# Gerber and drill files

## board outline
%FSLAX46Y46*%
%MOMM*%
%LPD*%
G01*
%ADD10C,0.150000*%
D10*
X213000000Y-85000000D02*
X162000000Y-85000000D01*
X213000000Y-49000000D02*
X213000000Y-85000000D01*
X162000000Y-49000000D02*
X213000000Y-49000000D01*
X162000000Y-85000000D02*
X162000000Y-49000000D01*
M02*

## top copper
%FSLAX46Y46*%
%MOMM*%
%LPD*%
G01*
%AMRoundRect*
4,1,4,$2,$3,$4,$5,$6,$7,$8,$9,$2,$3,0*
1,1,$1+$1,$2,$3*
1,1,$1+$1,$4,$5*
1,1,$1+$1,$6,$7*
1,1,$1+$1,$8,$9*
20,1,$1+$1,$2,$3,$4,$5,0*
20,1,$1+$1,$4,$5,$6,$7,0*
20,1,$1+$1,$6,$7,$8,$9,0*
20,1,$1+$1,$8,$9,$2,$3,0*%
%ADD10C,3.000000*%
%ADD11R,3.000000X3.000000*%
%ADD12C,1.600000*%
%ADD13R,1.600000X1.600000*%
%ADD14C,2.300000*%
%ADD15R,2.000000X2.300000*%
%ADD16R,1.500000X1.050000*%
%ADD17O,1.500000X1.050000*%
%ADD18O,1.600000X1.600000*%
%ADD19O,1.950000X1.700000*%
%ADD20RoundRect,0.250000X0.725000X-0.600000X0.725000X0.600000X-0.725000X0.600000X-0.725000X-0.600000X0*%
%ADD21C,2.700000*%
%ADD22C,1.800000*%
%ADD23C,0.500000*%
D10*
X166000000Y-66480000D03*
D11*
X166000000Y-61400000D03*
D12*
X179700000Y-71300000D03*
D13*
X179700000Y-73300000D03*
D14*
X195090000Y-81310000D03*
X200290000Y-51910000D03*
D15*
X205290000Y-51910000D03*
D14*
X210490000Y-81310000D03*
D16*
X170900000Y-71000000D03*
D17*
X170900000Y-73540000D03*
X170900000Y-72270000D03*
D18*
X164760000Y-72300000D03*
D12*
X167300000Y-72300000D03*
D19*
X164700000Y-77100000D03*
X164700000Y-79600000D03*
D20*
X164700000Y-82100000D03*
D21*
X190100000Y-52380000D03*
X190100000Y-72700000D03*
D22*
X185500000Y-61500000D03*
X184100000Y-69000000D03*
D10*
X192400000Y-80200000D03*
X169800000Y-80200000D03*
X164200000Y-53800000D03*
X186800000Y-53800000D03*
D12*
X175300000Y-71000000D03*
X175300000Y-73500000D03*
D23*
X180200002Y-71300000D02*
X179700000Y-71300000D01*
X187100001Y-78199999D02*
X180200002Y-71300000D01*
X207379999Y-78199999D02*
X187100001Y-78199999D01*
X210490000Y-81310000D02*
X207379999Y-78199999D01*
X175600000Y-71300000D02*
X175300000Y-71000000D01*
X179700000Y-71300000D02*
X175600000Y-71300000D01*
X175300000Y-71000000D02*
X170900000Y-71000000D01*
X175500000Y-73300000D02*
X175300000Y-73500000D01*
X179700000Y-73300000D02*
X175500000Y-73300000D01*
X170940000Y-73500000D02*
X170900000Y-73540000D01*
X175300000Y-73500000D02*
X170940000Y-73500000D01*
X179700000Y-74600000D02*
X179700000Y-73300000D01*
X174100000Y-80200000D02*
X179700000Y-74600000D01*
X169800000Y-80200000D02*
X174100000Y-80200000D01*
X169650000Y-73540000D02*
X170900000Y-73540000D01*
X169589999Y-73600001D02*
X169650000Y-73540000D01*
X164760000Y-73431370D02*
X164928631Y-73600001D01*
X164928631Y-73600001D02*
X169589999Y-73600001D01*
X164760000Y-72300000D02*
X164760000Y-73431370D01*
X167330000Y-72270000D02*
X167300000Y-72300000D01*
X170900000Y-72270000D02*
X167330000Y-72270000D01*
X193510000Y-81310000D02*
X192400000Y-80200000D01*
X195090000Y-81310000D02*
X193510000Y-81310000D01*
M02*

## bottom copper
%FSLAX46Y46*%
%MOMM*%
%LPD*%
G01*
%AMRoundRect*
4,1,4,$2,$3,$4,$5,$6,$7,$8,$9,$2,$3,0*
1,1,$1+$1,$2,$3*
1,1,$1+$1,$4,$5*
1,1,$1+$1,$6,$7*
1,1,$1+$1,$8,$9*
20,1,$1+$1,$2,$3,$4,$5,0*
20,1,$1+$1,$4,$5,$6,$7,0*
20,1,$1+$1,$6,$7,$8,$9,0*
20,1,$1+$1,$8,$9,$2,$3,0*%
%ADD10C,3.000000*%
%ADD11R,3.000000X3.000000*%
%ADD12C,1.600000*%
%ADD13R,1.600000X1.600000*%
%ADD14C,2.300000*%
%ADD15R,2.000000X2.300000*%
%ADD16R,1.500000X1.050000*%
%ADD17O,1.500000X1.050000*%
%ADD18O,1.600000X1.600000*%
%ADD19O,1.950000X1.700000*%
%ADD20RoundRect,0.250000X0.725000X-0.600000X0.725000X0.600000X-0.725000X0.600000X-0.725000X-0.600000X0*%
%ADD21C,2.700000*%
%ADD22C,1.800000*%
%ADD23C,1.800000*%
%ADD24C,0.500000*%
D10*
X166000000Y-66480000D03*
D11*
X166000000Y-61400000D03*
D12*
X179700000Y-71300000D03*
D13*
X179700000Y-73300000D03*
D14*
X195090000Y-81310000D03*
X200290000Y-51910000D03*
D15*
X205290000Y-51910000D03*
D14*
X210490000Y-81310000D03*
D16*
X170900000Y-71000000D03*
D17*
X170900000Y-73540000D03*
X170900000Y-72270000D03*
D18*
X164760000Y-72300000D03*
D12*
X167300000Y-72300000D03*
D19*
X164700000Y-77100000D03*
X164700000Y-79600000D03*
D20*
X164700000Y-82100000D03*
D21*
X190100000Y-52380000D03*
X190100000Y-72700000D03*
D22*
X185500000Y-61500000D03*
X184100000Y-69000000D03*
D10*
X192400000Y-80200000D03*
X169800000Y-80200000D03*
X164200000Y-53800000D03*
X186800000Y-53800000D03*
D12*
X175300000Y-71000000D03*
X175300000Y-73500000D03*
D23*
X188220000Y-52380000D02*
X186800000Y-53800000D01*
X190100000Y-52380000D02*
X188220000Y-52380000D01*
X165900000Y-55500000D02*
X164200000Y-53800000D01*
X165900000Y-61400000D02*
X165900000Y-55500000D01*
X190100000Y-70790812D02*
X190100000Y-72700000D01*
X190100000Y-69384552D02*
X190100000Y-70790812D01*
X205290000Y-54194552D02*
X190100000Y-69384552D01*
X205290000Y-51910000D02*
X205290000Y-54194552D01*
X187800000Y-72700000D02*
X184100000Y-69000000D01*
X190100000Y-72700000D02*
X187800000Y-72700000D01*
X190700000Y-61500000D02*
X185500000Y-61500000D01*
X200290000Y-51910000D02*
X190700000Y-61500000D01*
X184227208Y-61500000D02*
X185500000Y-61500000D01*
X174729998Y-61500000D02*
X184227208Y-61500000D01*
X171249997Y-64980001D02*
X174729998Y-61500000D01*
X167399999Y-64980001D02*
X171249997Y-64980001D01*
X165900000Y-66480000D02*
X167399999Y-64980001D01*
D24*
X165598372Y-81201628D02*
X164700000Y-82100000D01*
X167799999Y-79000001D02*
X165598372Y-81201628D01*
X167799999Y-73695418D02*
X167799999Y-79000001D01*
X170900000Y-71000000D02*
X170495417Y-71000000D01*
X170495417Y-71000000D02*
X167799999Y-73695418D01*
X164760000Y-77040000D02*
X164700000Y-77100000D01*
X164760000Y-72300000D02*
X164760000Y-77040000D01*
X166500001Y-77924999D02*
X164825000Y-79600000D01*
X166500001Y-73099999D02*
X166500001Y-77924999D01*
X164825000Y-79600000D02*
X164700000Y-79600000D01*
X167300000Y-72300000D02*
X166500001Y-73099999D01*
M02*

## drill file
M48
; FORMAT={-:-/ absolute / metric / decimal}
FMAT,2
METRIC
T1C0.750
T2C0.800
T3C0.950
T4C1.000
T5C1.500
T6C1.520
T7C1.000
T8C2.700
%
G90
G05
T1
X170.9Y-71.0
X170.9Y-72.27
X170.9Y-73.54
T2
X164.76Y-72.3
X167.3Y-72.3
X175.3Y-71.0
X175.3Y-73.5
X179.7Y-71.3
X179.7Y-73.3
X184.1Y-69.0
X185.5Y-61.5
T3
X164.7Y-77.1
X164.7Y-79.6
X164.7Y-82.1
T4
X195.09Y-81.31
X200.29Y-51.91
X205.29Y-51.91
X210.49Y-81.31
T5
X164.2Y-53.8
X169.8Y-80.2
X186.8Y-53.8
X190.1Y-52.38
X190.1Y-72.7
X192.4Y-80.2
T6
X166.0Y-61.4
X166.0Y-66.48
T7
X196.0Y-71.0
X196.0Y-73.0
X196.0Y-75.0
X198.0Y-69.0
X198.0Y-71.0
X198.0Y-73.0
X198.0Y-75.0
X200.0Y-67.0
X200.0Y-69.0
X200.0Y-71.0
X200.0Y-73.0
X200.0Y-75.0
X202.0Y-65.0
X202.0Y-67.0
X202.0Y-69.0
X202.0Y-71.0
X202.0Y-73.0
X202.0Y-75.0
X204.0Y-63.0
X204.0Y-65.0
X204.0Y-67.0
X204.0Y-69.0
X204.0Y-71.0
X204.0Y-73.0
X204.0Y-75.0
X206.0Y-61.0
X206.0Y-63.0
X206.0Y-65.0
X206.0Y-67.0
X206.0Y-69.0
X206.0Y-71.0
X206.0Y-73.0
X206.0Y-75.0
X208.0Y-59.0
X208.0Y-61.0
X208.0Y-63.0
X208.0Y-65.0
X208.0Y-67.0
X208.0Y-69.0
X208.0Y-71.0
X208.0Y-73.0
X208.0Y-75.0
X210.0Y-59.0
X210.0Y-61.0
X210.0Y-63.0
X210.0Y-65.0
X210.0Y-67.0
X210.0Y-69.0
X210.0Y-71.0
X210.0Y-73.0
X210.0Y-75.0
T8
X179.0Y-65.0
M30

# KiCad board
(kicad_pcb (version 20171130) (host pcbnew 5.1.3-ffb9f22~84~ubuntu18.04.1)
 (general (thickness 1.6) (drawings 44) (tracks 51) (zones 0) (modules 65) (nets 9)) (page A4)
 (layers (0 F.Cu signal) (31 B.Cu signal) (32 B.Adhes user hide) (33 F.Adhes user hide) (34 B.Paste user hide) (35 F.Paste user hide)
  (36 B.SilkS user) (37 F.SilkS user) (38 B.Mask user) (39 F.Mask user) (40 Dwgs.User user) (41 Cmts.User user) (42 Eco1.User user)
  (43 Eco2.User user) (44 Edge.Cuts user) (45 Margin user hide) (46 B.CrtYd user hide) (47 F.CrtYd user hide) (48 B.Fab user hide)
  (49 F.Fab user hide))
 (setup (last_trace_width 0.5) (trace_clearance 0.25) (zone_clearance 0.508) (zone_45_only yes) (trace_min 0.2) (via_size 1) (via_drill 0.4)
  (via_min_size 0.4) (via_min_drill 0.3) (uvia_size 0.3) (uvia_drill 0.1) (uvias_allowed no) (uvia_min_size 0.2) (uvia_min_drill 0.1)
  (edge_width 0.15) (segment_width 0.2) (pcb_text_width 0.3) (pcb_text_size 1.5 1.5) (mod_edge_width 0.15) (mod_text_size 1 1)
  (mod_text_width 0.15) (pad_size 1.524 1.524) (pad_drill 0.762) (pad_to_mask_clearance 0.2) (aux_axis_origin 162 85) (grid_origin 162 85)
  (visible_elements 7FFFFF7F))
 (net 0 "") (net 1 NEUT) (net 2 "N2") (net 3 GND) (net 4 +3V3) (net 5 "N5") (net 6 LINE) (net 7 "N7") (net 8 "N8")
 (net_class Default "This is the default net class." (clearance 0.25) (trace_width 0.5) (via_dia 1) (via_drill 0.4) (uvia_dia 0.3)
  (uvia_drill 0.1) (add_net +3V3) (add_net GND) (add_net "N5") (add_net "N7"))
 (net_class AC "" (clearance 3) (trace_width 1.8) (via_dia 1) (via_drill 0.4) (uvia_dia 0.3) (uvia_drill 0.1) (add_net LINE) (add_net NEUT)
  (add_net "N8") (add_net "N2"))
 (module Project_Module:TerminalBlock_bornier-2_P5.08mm (layer F.Cu) (at 166 61.4 270)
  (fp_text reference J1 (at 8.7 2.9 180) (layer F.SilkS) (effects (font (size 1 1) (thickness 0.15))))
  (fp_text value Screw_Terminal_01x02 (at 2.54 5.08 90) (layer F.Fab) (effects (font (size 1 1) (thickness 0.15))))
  (pad 2 thru_hole circle (at 5.08 0 270) (size 3 3) (drill 1.52) (layers *.Cu *.Mask) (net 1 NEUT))
  (pad 1 thru_hole rect (at 0 0 270) (size 3 3) (drill 1.52) (layers *.Cu *.Mask) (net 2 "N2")))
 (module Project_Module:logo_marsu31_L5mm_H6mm (layer B.Cu) (at 173.8 80.9 180)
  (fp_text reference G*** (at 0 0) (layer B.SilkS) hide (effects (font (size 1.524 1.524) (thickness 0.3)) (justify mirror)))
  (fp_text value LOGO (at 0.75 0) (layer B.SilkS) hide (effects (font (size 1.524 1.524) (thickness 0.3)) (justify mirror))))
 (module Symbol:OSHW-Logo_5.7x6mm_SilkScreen (layer B.Cu) (at 202.9 80.9 180)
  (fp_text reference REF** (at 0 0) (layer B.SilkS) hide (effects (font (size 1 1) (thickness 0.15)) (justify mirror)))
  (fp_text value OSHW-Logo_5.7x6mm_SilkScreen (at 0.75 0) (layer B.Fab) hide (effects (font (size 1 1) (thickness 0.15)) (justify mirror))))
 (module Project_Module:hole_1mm (layer F.Cu) (at 210 75)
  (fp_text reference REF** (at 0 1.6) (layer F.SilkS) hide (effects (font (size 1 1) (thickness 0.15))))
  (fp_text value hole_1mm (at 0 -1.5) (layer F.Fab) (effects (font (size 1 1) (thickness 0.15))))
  (pad "" np_thru_hole circle (at 0 0) (size 1 1) (drill 1) (layers *.Cu *.Mask)))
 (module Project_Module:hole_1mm (layer F.Cu) (at 208 75)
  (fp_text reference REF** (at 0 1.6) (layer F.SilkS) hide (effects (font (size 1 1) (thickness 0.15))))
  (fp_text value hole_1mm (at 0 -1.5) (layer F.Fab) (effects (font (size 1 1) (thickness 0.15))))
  (pad "" np_thru_hole circle (at 0 0) (size 1 1) (drill 1) (layers *.Cu *.Mask)))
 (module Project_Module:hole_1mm (layer F.Cu) (at 206 75)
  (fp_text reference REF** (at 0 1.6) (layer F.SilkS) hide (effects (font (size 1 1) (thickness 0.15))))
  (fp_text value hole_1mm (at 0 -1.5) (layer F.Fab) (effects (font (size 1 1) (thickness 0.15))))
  (pad "" np_thru_hole circle (at 0 0) (size 1 1) (drill 1) (layers *.Cu *.Mask)))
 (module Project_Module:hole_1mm (layer F.Cu) (at 204 75)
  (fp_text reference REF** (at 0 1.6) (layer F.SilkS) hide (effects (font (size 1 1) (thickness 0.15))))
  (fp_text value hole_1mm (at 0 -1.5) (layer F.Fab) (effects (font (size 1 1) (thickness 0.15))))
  (pad "" np_thru_hole circle (at 0 0) (size 1 1) (drill 1) (layers *.Cu *.Mask)))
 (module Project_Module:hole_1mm (layer F.Cu) (at 202 75)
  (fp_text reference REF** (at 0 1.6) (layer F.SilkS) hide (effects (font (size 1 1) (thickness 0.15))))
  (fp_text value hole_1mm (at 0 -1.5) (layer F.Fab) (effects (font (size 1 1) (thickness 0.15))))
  (pad "" np_thru_hole circle (at 0 0) (size 1 1) (drill 1) (layers *.Cu *.Mask)))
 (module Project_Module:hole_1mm (layer F.Cu) (at 200 75)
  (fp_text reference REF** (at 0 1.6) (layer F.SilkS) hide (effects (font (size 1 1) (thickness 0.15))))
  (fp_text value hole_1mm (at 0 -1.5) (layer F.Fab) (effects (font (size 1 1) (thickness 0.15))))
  (pad "" np_thru_hole circle (at 0 0) (size 1 1) (drill 1) (layers *.Cu *.Mask)))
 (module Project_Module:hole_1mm (layer F.Cu) (at 198 75)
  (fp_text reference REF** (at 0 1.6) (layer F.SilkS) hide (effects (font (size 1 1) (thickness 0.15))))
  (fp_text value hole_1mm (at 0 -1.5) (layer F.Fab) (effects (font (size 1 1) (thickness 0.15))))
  (pad "" np_thru_hole circle (at 0 0) (size 1 1) (drill 1) (layers *.Cu *.Mask)))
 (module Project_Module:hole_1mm (layer F.Cu) (at 196 75)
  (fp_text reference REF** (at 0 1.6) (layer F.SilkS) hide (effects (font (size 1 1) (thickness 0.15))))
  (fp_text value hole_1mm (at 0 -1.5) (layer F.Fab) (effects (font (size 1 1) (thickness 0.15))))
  (pad "" np_thru_hole circle (at 0 0) (size 1 1) (drill 1) (layers *.Cu *.Mask)))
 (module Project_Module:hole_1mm (layer F.Cu) (at 210 73)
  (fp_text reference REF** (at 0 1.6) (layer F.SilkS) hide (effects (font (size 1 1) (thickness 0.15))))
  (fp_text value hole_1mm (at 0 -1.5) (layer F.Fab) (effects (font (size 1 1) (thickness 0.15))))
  (pad "" np_thru_hole circle (at 0 0) (size 1 1) (drill 1) (layers *.Cu *.Mask)))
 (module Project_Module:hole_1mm (layer F.Cu) (at 208 73)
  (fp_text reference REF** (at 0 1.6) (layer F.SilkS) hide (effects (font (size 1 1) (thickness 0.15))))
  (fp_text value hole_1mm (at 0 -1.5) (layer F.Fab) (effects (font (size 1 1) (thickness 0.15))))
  (pad "" np_thru_hole circle (at 0 0) (size 1 1) (drill 1) (layers *.Cu *.Mask)))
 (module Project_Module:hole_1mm (layer F.Cu) (at 206 73)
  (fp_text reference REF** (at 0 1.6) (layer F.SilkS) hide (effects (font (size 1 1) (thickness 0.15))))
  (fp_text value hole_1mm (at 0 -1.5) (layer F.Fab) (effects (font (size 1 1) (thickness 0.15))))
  (pad "" np_thru_hole circle (at 0 0) (size 1 1) (drill 1) (layers *.Cu *.Mask)))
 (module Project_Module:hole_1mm (layer F.Cu) (at 204 73)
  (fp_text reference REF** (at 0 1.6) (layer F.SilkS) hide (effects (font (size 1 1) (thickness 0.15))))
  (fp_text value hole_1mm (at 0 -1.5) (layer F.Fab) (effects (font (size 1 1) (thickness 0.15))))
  (pad "" np_thru_hole circle (at 0 0) (size 1 1) (drill 1) (layers *.Cu *.Mask)))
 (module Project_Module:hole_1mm (layer F.Cu) (at 202 73)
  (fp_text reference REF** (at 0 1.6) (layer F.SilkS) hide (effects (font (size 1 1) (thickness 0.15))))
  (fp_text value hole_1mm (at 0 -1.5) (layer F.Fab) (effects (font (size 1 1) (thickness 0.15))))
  (pad "" np_thru_hole circle (at 0 0) (size 1 1) (drill 1) (layers *.Cu *.Mask)))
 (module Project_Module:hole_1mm (layer F.Cu) (at 200 73)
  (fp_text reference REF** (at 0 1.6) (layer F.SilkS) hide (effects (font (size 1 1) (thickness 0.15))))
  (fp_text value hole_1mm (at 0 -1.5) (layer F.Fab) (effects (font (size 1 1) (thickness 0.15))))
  (pad "" np_thru_hole circle (at 0 0) (size 1 1) (drill 1) (layers *.Cu *.Mask)))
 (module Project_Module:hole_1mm (layer F.Cu) (at 198 73)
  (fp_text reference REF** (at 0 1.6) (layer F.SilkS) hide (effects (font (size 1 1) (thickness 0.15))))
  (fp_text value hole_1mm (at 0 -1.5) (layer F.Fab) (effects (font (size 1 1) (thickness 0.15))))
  (pad "" np_thru_hole circle (at 0 0) (size 1 1) (drill 1) (layers *.Cu *.Mask)))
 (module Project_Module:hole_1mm (layer F.Cu) (at 196 73)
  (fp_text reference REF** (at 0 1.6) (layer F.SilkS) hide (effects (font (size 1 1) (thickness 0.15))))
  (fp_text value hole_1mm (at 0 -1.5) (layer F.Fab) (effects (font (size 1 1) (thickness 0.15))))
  (pad "" np_thru_hole circle (at 0 0) (size 1 1) (drill 1) (layers *.Cu *.Mask)))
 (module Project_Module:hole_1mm (layer F.Cu) (at 210 71)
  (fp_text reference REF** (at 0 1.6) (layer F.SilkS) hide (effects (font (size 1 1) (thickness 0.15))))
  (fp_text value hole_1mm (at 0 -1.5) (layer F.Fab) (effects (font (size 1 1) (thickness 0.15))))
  (pad "" np_thru_hole circle (at 0 0) (size 1 1) (drill 1) (layers *.Cu *.Mask)))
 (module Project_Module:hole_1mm (layer F.Cu) (at 208 71)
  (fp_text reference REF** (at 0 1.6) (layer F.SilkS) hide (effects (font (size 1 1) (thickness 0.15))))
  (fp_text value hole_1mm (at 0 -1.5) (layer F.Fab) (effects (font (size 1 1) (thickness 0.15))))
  (pad "" np_thru_hole circle (at 0 0) (size 1 1) (drill 1) (layers *.Cu *.Mask)))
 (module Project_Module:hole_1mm (layer F.Cu) (at 206 71)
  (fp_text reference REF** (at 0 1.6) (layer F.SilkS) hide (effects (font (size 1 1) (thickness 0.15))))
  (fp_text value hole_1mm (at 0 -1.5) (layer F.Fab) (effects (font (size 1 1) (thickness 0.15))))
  (pad "" np_thru_hole circle (at 0 0) (size 1 1) (drill 1) (layers *.Cu *.Mask)))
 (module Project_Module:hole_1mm (layer F.Cu) (at 204 71)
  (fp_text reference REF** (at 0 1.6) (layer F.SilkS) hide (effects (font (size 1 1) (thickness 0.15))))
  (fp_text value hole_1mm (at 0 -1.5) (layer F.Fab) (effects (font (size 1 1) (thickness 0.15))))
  (pad "" np_thru_hole circle (at 0 0) (size 1 1) (drill 1) (layers *.Cu *.Mask)))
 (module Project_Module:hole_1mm (layer F.Cu) (at 202 71)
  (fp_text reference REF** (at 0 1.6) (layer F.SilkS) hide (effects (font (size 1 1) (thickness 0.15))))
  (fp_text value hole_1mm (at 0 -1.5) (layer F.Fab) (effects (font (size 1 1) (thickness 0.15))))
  (pad "" np_thru_hole circle (at 0 0) (size 1 1) (drill 1) (layers *.Cu *.Mask)))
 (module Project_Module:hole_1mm (layer F.Cu) (at 200 71)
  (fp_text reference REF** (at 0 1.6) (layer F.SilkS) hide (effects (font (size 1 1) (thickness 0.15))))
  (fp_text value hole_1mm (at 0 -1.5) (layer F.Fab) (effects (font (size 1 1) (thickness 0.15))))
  (pad "" np_thru_hole circle (at 0 0) (size 1 1) (drill 1) (layers *.Cu *.Mask)))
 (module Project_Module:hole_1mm (layer F.Cu) (at 198 71)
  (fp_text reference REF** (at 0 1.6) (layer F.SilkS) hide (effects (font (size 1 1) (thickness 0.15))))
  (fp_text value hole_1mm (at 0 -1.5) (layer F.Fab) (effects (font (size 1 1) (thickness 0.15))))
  (pad "" np_thru_hole circle (at 0 0) (size 1 1) (drill 1) (layers *.Cu *.Mask)))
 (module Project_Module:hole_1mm (layer F.Cu) (at 196 71)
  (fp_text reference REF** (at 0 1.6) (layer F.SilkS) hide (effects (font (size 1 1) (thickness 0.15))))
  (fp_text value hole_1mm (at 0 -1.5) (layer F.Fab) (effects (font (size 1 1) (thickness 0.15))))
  (pad "" np_thru_hole circle (at 0 0) (size 1 1) (drill 1) (layers *.Cu *.Mask)))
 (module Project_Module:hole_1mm (layer F.Cu) (at 210 69)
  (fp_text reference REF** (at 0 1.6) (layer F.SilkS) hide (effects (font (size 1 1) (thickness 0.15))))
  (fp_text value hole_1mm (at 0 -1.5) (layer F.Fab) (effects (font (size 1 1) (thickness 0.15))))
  (pad "" np_thru_hole circle (at 0 0) (size 1 1) (drill 1) (layers *.Cu *.Mask)))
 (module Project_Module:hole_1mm (layer F.Cu) (at 208 69)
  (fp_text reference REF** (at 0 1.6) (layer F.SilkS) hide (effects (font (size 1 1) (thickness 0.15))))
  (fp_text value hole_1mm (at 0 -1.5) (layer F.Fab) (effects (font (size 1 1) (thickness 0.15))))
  (pad "" np_thru_hole circle (at 0 0) (size 1 1) (drill 1) (layers *.Cu *.Mask)))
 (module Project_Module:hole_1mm (layer F.Cu) (at 206 69)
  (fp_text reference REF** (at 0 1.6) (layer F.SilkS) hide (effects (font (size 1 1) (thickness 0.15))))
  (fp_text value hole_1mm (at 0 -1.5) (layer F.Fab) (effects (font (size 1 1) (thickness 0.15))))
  (pad "" np_thru_hole circle (at 0 0) (size 1 1) (drill 1) (layers *.Cu *.Mask)))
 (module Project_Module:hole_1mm (layer F.Cu) (at 204 69)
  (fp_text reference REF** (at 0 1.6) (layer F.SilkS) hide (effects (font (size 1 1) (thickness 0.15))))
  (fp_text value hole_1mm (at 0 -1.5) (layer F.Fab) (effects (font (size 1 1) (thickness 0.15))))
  (pad "" np_thru_hole circle (at 0 0) (size 1 1) (drill 1) (layers *.Cu *.Mask)))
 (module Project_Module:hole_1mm (layer F.Cu) (at 202 69)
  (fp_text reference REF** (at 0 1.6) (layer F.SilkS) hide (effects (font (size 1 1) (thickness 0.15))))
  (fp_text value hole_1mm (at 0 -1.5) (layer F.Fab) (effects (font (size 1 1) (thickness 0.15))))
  (pad "" np_thru_hole circle (at 0 0) (size 1 1) (drill 1) (layers *.Cu *.Mask)))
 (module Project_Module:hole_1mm (layer F.Cu) (at 200 69)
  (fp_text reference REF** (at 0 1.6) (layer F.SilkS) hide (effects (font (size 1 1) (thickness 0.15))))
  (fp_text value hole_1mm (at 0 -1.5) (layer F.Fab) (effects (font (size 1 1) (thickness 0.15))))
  (pad "" np_thru_hole circle (at 0 0) (size 1 1) (drill 1) (layers *.Cu *.Mask)))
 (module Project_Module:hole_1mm (layer F.Cu) (at 198 69)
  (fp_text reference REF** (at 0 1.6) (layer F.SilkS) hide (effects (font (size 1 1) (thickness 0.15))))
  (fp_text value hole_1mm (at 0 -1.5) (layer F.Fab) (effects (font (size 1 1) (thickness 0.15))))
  (pad "" np_thru_hole circle (at 0 0) (size 1 1) (drill 1) (layers *.Cu *.Mask)))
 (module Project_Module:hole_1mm (layer F.Cu) (at 210 67)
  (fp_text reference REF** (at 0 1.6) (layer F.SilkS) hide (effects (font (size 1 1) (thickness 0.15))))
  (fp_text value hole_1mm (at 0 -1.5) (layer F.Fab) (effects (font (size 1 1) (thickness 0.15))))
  (pad "" np_thru_hole circle (at 0 0) (size 1 1) (drill 1) (layers *.Cu *.Mask)))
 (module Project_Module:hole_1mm (layer F.Cu) (at 208 67)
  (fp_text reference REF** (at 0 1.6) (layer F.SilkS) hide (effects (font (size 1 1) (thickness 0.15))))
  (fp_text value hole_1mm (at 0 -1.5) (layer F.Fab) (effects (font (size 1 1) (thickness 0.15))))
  (pad "" np_thru_hole circle (at 0 0) (size 1 1) (drill 1) (layers *.Cu *.Mask)))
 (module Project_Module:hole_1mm (layer F.Cu) (at 206 67)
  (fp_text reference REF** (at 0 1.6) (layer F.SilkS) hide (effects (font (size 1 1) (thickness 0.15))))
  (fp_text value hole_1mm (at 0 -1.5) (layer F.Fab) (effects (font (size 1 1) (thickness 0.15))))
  (pad "" np_thru_hole circle (at 0 0) (size 1 1) (drill 1) (layers *.Cu *.Mask)))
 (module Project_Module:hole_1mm (layer F.Cu) (at 204 67)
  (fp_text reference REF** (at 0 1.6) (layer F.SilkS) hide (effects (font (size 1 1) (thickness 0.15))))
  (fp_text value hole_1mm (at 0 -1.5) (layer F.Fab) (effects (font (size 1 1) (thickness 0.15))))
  (pad "" np_thru_hole circle (at 0 0) (size 1 1) (drill 1) (layers *.Cu *.Mask)))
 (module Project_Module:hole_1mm (layer F.Cu) (at 202 67)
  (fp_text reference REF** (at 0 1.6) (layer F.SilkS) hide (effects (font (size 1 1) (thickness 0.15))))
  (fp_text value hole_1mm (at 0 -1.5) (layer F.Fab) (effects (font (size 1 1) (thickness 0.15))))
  (pad "" np_thru_hole circle (at 0 0) (size 1 1) (drill 1) (layers *.Cu *.Mask)))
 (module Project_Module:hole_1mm (layer F.Cu) (at 200 67)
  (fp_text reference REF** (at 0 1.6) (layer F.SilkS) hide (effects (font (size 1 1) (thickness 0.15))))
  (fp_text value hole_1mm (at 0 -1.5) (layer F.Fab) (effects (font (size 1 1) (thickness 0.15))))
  (pad "" np_thru_hole circle (at 0 0) (size 1 1) (drill 1) (layers *.Cu *.Mask)))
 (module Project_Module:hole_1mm (layer F.Cu) (at 210 65)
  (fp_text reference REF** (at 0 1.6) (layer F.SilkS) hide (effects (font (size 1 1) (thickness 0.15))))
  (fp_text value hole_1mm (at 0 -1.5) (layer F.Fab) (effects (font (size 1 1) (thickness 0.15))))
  (pad "" np_thru_hole circle (at 0 0) (size 1 1) (drill 1) (layers *.Cu *.Mask)))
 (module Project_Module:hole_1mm (layer F.Cu) (at 208 65)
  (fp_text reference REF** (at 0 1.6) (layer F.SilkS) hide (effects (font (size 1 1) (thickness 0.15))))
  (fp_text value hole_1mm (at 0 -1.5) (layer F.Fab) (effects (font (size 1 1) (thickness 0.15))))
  (pad "" np_thru_hole circle (at 0 0) (size 1 1) (drill 1) (layers *.Cu *.Mask)))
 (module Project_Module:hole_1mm (layer F.Cu) (at 206 65)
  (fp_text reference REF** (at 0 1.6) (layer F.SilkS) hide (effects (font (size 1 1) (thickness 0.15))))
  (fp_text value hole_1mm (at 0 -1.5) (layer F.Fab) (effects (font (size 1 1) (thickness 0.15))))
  (pad "" np_thru_hole circle (at 0 0) (size 1 1) (drill 1) (layers *.Cu *.Mask)))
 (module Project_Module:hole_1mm (layer F.Cu) (at 204 65)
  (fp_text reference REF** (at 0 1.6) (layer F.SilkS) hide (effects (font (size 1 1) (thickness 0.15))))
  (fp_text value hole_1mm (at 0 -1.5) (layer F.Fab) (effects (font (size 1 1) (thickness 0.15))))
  (pad "" np_thru_hole circle (at 0 0) (size 1 1) (drill 1) (layers *.Cu *.Mask)))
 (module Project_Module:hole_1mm (layer F.Cu) (at 202 65)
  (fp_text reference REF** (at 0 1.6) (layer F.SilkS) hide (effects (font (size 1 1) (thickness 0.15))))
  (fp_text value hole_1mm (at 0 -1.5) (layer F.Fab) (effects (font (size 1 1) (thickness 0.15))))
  (pad "" np_thru_hole circle (at 0 0) (size 1 1) (drill 1) (layers *.Cu *.Mask)))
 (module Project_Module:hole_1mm (layer F.Cu) (at 210 63)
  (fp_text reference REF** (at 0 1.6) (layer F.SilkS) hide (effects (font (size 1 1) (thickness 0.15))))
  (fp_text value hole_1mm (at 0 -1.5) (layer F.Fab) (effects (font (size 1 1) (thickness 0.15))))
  (pad "" np_thru_hole circle (at 0 0) (size 1 1) (drill 1) (layers *.Cu *.Mask)))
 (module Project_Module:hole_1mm (layer F.Cu) (at 208 63)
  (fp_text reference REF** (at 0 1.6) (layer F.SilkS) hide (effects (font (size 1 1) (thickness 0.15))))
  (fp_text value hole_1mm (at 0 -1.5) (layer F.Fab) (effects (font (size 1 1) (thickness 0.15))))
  (pad "" np_thru_hole circle (at 0 0) (size 1 1) (drill 1) (layers *.Cu *.Mask)))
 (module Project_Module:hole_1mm (layer F.Cu) (at 206 63)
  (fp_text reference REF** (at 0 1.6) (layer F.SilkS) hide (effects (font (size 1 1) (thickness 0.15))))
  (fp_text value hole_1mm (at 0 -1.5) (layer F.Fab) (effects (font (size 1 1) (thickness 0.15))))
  (pad "" np_thru_hole circle (at 0 0) (size 1 1) (drill 1) (layers *.Cu *.Mask)))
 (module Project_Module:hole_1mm (layer F.Cu) (at 204 63)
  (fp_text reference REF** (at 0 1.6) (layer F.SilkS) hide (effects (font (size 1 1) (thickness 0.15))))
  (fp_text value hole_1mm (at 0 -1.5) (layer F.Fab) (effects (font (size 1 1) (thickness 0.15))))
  (pad "" np_thru_hole circle (at 0 0) (size 1 1) (drill 1) (layers *.Cu *.Mask)))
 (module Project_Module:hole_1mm (layer F.Cu) (at 210 61)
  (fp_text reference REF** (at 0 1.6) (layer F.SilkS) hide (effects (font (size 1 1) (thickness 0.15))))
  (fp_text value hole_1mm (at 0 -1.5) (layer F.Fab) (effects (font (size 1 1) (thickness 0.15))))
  (pad "" np_thru_hole circle (at 0 0) (size 1 1) (drill 1) (layers *.Cu *.Mask)))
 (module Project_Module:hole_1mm (layer F.Cu) (at 208 61)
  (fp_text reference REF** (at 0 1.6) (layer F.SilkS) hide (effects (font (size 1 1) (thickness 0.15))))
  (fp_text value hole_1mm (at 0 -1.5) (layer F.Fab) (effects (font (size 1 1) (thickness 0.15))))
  (pad "" np_thru_hole circle (at 0 0) (size 1 1) (drill 1) (layers *.Cu *.Mask)))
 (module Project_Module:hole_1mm (layer F.Cu) (at 206 61)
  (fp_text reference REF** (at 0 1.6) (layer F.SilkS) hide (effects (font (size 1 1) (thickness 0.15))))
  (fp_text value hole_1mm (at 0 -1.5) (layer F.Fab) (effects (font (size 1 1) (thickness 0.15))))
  (pad "" np_thru_hole circle (at 0 0) (size 1 1) (drill 1) (layers *.Cu *.Mask)))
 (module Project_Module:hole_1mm (layer F.Cu) (at 210 59)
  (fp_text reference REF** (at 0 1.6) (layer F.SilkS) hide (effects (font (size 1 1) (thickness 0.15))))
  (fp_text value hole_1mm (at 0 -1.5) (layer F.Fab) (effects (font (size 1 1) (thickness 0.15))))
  (pad "" np_thru_hole circle (at 0 0) (size 1 1) (drill 1) (layers *.Cu *.Mask)))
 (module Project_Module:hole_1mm (layer F.Cu) (at 208 59)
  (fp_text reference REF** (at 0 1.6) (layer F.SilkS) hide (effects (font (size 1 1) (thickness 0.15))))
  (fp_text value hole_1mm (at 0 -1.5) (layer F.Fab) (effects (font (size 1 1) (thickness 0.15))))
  (pad "" np_thru_hole circle (at 0 0) (size 1 1) (drill 1) (layers *.Cu *.Mask)))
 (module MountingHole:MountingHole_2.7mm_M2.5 (layer F.Cu) (at 179 65)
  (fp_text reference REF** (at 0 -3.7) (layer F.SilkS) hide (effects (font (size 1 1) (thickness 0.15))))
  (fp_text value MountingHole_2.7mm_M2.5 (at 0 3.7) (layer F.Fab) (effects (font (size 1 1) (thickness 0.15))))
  (pad 1 np_thru_hole circle (at 0 0) (size 2.7 2.7) (drill 2.7) (layers *.Cu *.Mask)))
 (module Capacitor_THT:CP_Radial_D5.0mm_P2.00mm (layer F.Cu) (at 179.7 73.3 90)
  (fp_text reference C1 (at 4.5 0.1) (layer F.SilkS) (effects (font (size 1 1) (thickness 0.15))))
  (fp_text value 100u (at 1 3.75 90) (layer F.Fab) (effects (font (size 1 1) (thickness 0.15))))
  (pad 2 thru_hole circle (at 2 0 90) (size 1.6 1.6) (drill 0.8) (layers *.Cu *.Mask) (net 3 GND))
  (pad 1 thru_hole rect (at 0 0 90) (size 1.6 1.6) (drill 0.8) (layers *.Cu *.Mask) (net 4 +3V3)))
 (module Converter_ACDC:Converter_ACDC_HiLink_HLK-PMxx (layer F.Cu) (at 205.29 51.91 270)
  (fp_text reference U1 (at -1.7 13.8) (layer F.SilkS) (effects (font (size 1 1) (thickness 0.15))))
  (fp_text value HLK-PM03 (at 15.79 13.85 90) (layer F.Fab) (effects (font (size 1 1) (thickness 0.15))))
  (pad 4 thru_hole circle (at 29.4 10.2 270) (size 2.3 2.3) (drill 1) (layers *.Cu *.Mask) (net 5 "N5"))
  (pad 2 thru_hole circle (at 0 5 270) (size 2.3 2.3) (drill 1) (layers *.Cu *.Mask) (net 1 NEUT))
  (pad 1 thru_hole rect (at 0 0 270) (size 2.3 2) (drill 1) (layers *.Cu *.Mask) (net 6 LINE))
  (pad 3 thru_hole circle (at 29.4 -5.2 270) (size 2.3 2.3) (drill 1) (layers *.Cu *.Mask) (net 3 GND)))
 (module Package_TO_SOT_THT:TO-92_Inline (layer F.Cu) (at 170.9 71 270)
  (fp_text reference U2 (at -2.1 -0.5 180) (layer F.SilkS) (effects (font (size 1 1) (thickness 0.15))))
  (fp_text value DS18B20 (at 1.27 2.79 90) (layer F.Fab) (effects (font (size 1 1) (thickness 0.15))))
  (pad 1 thru_hole rect (at 0 0 270) (size 1.05 1.5) (drill 0.75) (layers *.Cu *.Mask) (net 3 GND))
  (pad 3 thru_hole oval (at 2.54 0 270) (size 1.05 1.5) (drill 0.75) (layers *.Cu *.Mask) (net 4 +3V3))
  (pad 2 thru_hole oval (at 1.27 0 270) (size 1.05 1.5) (drill 0.75) (layers *.Cu *.Mask) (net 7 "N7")))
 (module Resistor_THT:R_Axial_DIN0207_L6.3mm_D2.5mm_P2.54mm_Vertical (layer F.Cu) (at 167.3 72.3 180)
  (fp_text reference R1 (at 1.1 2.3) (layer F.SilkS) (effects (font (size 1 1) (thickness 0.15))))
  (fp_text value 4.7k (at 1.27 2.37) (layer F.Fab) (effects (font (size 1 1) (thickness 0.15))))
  (pad 2 thru_hole oval (at 2.54 0 180) (size 1.6 1.6) (drill 0.8) (layers *.Cu *.Mask) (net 4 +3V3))
  (pad 1 thru_hole circle (at 0 0 180) (size 1.6 1.6) (drill 0.8) (layers *.Cu *.Mask) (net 7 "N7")))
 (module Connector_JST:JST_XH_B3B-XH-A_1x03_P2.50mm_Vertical (layer F.Cu) (at 164.7 82.1 90)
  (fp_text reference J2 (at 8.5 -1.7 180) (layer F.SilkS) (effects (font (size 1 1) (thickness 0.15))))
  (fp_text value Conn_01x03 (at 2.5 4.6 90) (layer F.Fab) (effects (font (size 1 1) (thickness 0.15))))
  (pad 3 thru_hole oval (at 5 0 90) (size 1.7 1.95) (drill 0.95) (layers *.Cu *.Mask) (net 4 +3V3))
  (pad 2 thru_hole oval (at 2.5 0 90) (size 1.7 1.95) (drill 0.95) (layers *.Cu *.Mask) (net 7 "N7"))
  (pad 1 thru_hole roundrect (at 0 0 90) (size 1.7 1.95) (drill 0.95) (layers *.Cu *.Mask) (roundrect_rratio 0.147059) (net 3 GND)))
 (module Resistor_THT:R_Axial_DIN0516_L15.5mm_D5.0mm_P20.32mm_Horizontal (layer F.Cu) (at 190.1 72.7 90)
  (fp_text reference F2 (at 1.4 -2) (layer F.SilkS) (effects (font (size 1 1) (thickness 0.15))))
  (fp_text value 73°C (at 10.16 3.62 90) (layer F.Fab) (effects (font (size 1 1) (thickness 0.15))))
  (pad 2 thru_hole circle (at 20.32 0 90) (size 2.7 2.7) (drill 1.5) (layers *.Cu *.Mask) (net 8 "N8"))
  (pad 1 thru_hole circle (at 0 0 90) (size 2.7 2.7) (drill 1.5) (layers *.Cu *.Mask) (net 6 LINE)))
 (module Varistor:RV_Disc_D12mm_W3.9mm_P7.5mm (layer F.Cu) (at 184.1 69 90)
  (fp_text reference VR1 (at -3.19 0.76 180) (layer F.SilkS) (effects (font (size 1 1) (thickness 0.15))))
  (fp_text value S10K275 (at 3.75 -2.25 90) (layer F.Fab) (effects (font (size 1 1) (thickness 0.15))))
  (pad 2 thru_hole circle (at 7.5 1.4 90) (size 1.8 1.8) (drill 0.8) (layers *.Cu *.Mask) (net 1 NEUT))
  (pad 1 thru_hole circle (at 0 0 90) (size 1.8 1.8) (drill 0.8) (layers *.Cu *.Mask) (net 6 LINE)))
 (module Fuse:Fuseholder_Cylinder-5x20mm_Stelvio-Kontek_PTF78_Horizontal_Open (layer F.Cu) (at 169.8 80.2)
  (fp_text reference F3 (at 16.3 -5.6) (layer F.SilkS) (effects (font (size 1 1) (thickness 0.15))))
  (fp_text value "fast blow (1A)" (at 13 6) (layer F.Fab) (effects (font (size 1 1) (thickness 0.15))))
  (pad 2 thru_hole circle (at 22.6 0) (size 3 3) (drill 1.5) (layers *.Cu *.Mask) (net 5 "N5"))
  (pad 1 thru_hole circle (at 0 0) (size 3 3) (drill 1.5) (layers *.Cu *.Mask) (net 4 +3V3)))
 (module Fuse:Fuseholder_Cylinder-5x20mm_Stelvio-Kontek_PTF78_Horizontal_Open (layer F.Cu) (at 186.8 53.8 180)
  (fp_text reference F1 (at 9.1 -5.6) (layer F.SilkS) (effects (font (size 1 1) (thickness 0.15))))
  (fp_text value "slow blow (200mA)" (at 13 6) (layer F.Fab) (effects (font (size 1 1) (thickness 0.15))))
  (pad 2 thru_hole circle (at 22.6 0 180) (size 3 3) (drill 1.5) (layers *.Cu *.Mask) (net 2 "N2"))
  (pad 1 thru_hole circle (at 0 0 180) (size 3 3) (drill 1.5) (layers *.Cu *.Mask) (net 8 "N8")))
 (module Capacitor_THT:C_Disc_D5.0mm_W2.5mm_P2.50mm (layer F.Cu) (at 175.3 73.5 90)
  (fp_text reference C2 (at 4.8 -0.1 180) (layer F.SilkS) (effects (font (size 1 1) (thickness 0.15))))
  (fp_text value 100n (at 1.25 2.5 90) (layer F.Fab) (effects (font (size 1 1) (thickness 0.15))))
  (pad 2 thru_hole circle (at 2.5 0 90) (size 1.6 1.6) (drill 0.8) (layers *.Cu *.Mask) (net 3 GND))
  (pad 1 thru_hole circle (at 0 0 90) (size 1.6 1.6) (drill 0.8) (layers *.Cu *.Mask) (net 4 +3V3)))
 (gr_line (start 213 85) (end 162 85) (layer Edge.Cuts) (width 0.15))
 (gr_line (start 213 49) (end 213 85) (layer Edge.Cuts) (width 0.15))
 (gr_line (start 162 49) (end 213 49) (layer Edge.Cuts) (width 0.15))
 (gr_line (start 162 85) (end 162 49) (layer Edge.Cuts) (width 0.15))
 (segment (start 188.22 52.38) (end 186.8 53.8) (width 1.8) (layer B.Cu) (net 8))
 (segment (start 190.1 52.38) (end 188.22 52.38) (width 1.8) (layer B.Cu) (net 8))
 (segment (start 165.9 55.5) (end 164.2 53.8) (width 1.8) (layer B.Cu) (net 2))
 (segment (start 165.9 61.4) (end 165.9 55.5) (width 1.8) (layer B.Cu) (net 2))
 (segment (start 190.1 70.790812) (end 190.1 72.7) (width 1.8) (layer B.Cu) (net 6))
 (segment (start 190.1 69.384552) (end 190.1 70.790812) (width 1.8) (layer B.Cu) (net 6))
 (segment (start 205.29 54.194552) (end 190.1 69.384552) (width 1.8) (layer B.Cu) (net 6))
 (segment (start 205.29 51.91) (end 205.29 54.194552) (width 1.8) (layer B.Cu) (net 6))
 (segment (start 187.8 72.7) (end 184.1 69) (width 1.8) (layer B.Cu) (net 6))
 (segment (start 190.1 72.7) (end 187.8 72.7) (width 1.8) (layer B.Cu) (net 6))
 (segment (start 190.7 61.5) (end 185.5 61.5) (width 1.8) (layer B.Cu) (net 1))
 (segment (start 200.29 51.91) (end 190.7 61.5) (width 1.8) (layer B.Cu) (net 1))
 (segment (start 184.227208 61.5) (end 185.5 61.5) (width 1.8) (layer B.Cu) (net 1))
 (segment (start 174.729998 61.5) (end 184.227208 61.5) (width 1.8) (layer B.Cu) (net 1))
 (segment (start 171.249997 64.980001) (end 174.729998 61.5) (width 1.8) (layer B.Cu) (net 1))
 (segment (start 167.399999 64.980001) (end 171.249997 64.980001) (width 1.8) (layer B.Cu) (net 1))
 (segment (start 165.9 66.48) (end 167.399999 64.980001) (width 1.8) (layer B.Cu) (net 1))
 (segment (start 180.200002 71.3) (end 179.7 71.3) (width 0.5) (layer F.Cu) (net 3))
 (segment (start 187.100001 78.199999) (end 180.200002 71.3) (width 0.5) (layer F.Cu) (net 3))
 (segment (start 207.379999 78.199999) (end 187.100001 78.199999) (width 0.5) (layer F.Cu) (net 3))
 (segment (start 210.49 81.31) (end 207.379999 78.199999) (width 0.5) (layer F.Cu) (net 3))
 (segment (start 175.6 71.3) (end 175.3 71) (width 0.5) (layer F.Cu) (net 3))
 (segment (start 179.7 71.3) (end 175.6 71.3) (width 0.5) (layer F.Cu) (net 3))
 (segment (start 175.3 71) (end 170.9 71) (width 0.5) (layer F.Cu) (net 3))
 (segment (start 165.598372 81.201628) (end 164.7 82.1) (width 0.5) (layer B.Cu) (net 3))
 (segment (start 167.799999 79.000001) (end 165.598372 81.201628) (width 0.5) (layer B.Cu) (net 3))
 (segment (start 167.799999 73.695418) (end 167.799999 79.000001) (width 0.5) (layer B.Cu) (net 3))
 (segment (start 170.9 71) (end 170.495417 71) (width 0.5) (layer B.Cu) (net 3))
 (segment (start 170.495417 71) (end 167.799999 73.695418) (width 0.5) (layer B.Cu) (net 3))
 (segment (start 175.5 73.3) (end 175.3 73.5) (width 0.5) (layer F.Cu) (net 4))
 (segment (start 179.7 73.3) (end 175.5 73.3) (width 0.5) (layer F.Cu) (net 4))
 (segment (start 170.94 73.5) (end 170.9 73.54) (width 0.5) (layer F.Cu) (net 4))
 (segment (start 175.3 73.5) (end 170.94 73.5) (width 0.5) (layer F.Cu) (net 4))
 (segment (start 179.7 74.6) (end 179.7 73.3) (width 0.5) (layer F.Cu) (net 4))
 (segment (start 174.1 80.2) (end 179.7 74.6) (width 0.5) (layer F.Cu) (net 4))
 (segment (start 169.8 80.2) (end 174.1 80.2) (width 0.5) (layer F.Cu) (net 4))
 (segment (start 169.65 73.54) (end 170.9 73.54) (width 0.5) (layer F.Cu) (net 4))
 (segment (start 169.589999 73.600001) (end 169.65 73.54) (width 0.5) (layer F.Cu) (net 4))
 (segment (start 164.76 73.43137) (end 164.928631 73.600001) (width 0.5) (layer F.Cu) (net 4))
 (segment (start 164.928631 73.600001) (end 169.589999 73.600001) (width 0.5) (layer F.Cu) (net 4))
 (segment (start 164.76 72.3) (end 164.76 73.43137) (width 0.5) (layer F.Cu) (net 4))
 (segment (start 164.76 77.04) (end 164.7 77.1) (width 0.5) (layer B.Cu) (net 4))
 (segment (start 164.76 72.3) (end 164.76 77.04) (width 0.5) (layer B.Cu) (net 4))
 (segment (start 167.33 72.27) (end 167.3 72.3) (width 0.5) (layer F.Cu) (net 7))
 (segment (start 170.9 72.27) (end 167.33 72.27) (width 0.5) (layer F.Cu) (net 7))
 (segment (start 166.500001 77.924999) (end 164.825 79.6) (width 0.5) (layer B.Cu) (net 7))
 (segment (start 166.500001 73.099999) (end 166.500001 77.924999) (width 0.5) (layer B.Cu) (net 7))
 (segment (start 164.825 79.6) (end 164.7 79.6) (width 0.5) (layer B.Cu) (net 7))
 (segment (start 167.3 72.3) (end 166.500001 73.099999) (width 0.5) (layer B.Cu) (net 7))
 (segment (start 193.51 81.31) (end 192.4 80.2) (width 0.5) (layer F.Cu) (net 5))
 (segment (start 195.09 81.31) (end 193.51 81.31) (width 0.5) (layer F.Cu) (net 5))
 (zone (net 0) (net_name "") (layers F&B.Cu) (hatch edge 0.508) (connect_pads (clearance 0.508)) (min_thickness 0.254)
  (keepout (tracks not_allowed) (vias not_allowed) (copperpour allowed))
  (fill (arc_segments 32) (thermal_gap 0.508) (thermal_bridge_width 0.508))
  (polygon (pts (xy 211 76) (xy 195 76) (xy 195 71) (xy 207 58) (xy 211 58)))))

